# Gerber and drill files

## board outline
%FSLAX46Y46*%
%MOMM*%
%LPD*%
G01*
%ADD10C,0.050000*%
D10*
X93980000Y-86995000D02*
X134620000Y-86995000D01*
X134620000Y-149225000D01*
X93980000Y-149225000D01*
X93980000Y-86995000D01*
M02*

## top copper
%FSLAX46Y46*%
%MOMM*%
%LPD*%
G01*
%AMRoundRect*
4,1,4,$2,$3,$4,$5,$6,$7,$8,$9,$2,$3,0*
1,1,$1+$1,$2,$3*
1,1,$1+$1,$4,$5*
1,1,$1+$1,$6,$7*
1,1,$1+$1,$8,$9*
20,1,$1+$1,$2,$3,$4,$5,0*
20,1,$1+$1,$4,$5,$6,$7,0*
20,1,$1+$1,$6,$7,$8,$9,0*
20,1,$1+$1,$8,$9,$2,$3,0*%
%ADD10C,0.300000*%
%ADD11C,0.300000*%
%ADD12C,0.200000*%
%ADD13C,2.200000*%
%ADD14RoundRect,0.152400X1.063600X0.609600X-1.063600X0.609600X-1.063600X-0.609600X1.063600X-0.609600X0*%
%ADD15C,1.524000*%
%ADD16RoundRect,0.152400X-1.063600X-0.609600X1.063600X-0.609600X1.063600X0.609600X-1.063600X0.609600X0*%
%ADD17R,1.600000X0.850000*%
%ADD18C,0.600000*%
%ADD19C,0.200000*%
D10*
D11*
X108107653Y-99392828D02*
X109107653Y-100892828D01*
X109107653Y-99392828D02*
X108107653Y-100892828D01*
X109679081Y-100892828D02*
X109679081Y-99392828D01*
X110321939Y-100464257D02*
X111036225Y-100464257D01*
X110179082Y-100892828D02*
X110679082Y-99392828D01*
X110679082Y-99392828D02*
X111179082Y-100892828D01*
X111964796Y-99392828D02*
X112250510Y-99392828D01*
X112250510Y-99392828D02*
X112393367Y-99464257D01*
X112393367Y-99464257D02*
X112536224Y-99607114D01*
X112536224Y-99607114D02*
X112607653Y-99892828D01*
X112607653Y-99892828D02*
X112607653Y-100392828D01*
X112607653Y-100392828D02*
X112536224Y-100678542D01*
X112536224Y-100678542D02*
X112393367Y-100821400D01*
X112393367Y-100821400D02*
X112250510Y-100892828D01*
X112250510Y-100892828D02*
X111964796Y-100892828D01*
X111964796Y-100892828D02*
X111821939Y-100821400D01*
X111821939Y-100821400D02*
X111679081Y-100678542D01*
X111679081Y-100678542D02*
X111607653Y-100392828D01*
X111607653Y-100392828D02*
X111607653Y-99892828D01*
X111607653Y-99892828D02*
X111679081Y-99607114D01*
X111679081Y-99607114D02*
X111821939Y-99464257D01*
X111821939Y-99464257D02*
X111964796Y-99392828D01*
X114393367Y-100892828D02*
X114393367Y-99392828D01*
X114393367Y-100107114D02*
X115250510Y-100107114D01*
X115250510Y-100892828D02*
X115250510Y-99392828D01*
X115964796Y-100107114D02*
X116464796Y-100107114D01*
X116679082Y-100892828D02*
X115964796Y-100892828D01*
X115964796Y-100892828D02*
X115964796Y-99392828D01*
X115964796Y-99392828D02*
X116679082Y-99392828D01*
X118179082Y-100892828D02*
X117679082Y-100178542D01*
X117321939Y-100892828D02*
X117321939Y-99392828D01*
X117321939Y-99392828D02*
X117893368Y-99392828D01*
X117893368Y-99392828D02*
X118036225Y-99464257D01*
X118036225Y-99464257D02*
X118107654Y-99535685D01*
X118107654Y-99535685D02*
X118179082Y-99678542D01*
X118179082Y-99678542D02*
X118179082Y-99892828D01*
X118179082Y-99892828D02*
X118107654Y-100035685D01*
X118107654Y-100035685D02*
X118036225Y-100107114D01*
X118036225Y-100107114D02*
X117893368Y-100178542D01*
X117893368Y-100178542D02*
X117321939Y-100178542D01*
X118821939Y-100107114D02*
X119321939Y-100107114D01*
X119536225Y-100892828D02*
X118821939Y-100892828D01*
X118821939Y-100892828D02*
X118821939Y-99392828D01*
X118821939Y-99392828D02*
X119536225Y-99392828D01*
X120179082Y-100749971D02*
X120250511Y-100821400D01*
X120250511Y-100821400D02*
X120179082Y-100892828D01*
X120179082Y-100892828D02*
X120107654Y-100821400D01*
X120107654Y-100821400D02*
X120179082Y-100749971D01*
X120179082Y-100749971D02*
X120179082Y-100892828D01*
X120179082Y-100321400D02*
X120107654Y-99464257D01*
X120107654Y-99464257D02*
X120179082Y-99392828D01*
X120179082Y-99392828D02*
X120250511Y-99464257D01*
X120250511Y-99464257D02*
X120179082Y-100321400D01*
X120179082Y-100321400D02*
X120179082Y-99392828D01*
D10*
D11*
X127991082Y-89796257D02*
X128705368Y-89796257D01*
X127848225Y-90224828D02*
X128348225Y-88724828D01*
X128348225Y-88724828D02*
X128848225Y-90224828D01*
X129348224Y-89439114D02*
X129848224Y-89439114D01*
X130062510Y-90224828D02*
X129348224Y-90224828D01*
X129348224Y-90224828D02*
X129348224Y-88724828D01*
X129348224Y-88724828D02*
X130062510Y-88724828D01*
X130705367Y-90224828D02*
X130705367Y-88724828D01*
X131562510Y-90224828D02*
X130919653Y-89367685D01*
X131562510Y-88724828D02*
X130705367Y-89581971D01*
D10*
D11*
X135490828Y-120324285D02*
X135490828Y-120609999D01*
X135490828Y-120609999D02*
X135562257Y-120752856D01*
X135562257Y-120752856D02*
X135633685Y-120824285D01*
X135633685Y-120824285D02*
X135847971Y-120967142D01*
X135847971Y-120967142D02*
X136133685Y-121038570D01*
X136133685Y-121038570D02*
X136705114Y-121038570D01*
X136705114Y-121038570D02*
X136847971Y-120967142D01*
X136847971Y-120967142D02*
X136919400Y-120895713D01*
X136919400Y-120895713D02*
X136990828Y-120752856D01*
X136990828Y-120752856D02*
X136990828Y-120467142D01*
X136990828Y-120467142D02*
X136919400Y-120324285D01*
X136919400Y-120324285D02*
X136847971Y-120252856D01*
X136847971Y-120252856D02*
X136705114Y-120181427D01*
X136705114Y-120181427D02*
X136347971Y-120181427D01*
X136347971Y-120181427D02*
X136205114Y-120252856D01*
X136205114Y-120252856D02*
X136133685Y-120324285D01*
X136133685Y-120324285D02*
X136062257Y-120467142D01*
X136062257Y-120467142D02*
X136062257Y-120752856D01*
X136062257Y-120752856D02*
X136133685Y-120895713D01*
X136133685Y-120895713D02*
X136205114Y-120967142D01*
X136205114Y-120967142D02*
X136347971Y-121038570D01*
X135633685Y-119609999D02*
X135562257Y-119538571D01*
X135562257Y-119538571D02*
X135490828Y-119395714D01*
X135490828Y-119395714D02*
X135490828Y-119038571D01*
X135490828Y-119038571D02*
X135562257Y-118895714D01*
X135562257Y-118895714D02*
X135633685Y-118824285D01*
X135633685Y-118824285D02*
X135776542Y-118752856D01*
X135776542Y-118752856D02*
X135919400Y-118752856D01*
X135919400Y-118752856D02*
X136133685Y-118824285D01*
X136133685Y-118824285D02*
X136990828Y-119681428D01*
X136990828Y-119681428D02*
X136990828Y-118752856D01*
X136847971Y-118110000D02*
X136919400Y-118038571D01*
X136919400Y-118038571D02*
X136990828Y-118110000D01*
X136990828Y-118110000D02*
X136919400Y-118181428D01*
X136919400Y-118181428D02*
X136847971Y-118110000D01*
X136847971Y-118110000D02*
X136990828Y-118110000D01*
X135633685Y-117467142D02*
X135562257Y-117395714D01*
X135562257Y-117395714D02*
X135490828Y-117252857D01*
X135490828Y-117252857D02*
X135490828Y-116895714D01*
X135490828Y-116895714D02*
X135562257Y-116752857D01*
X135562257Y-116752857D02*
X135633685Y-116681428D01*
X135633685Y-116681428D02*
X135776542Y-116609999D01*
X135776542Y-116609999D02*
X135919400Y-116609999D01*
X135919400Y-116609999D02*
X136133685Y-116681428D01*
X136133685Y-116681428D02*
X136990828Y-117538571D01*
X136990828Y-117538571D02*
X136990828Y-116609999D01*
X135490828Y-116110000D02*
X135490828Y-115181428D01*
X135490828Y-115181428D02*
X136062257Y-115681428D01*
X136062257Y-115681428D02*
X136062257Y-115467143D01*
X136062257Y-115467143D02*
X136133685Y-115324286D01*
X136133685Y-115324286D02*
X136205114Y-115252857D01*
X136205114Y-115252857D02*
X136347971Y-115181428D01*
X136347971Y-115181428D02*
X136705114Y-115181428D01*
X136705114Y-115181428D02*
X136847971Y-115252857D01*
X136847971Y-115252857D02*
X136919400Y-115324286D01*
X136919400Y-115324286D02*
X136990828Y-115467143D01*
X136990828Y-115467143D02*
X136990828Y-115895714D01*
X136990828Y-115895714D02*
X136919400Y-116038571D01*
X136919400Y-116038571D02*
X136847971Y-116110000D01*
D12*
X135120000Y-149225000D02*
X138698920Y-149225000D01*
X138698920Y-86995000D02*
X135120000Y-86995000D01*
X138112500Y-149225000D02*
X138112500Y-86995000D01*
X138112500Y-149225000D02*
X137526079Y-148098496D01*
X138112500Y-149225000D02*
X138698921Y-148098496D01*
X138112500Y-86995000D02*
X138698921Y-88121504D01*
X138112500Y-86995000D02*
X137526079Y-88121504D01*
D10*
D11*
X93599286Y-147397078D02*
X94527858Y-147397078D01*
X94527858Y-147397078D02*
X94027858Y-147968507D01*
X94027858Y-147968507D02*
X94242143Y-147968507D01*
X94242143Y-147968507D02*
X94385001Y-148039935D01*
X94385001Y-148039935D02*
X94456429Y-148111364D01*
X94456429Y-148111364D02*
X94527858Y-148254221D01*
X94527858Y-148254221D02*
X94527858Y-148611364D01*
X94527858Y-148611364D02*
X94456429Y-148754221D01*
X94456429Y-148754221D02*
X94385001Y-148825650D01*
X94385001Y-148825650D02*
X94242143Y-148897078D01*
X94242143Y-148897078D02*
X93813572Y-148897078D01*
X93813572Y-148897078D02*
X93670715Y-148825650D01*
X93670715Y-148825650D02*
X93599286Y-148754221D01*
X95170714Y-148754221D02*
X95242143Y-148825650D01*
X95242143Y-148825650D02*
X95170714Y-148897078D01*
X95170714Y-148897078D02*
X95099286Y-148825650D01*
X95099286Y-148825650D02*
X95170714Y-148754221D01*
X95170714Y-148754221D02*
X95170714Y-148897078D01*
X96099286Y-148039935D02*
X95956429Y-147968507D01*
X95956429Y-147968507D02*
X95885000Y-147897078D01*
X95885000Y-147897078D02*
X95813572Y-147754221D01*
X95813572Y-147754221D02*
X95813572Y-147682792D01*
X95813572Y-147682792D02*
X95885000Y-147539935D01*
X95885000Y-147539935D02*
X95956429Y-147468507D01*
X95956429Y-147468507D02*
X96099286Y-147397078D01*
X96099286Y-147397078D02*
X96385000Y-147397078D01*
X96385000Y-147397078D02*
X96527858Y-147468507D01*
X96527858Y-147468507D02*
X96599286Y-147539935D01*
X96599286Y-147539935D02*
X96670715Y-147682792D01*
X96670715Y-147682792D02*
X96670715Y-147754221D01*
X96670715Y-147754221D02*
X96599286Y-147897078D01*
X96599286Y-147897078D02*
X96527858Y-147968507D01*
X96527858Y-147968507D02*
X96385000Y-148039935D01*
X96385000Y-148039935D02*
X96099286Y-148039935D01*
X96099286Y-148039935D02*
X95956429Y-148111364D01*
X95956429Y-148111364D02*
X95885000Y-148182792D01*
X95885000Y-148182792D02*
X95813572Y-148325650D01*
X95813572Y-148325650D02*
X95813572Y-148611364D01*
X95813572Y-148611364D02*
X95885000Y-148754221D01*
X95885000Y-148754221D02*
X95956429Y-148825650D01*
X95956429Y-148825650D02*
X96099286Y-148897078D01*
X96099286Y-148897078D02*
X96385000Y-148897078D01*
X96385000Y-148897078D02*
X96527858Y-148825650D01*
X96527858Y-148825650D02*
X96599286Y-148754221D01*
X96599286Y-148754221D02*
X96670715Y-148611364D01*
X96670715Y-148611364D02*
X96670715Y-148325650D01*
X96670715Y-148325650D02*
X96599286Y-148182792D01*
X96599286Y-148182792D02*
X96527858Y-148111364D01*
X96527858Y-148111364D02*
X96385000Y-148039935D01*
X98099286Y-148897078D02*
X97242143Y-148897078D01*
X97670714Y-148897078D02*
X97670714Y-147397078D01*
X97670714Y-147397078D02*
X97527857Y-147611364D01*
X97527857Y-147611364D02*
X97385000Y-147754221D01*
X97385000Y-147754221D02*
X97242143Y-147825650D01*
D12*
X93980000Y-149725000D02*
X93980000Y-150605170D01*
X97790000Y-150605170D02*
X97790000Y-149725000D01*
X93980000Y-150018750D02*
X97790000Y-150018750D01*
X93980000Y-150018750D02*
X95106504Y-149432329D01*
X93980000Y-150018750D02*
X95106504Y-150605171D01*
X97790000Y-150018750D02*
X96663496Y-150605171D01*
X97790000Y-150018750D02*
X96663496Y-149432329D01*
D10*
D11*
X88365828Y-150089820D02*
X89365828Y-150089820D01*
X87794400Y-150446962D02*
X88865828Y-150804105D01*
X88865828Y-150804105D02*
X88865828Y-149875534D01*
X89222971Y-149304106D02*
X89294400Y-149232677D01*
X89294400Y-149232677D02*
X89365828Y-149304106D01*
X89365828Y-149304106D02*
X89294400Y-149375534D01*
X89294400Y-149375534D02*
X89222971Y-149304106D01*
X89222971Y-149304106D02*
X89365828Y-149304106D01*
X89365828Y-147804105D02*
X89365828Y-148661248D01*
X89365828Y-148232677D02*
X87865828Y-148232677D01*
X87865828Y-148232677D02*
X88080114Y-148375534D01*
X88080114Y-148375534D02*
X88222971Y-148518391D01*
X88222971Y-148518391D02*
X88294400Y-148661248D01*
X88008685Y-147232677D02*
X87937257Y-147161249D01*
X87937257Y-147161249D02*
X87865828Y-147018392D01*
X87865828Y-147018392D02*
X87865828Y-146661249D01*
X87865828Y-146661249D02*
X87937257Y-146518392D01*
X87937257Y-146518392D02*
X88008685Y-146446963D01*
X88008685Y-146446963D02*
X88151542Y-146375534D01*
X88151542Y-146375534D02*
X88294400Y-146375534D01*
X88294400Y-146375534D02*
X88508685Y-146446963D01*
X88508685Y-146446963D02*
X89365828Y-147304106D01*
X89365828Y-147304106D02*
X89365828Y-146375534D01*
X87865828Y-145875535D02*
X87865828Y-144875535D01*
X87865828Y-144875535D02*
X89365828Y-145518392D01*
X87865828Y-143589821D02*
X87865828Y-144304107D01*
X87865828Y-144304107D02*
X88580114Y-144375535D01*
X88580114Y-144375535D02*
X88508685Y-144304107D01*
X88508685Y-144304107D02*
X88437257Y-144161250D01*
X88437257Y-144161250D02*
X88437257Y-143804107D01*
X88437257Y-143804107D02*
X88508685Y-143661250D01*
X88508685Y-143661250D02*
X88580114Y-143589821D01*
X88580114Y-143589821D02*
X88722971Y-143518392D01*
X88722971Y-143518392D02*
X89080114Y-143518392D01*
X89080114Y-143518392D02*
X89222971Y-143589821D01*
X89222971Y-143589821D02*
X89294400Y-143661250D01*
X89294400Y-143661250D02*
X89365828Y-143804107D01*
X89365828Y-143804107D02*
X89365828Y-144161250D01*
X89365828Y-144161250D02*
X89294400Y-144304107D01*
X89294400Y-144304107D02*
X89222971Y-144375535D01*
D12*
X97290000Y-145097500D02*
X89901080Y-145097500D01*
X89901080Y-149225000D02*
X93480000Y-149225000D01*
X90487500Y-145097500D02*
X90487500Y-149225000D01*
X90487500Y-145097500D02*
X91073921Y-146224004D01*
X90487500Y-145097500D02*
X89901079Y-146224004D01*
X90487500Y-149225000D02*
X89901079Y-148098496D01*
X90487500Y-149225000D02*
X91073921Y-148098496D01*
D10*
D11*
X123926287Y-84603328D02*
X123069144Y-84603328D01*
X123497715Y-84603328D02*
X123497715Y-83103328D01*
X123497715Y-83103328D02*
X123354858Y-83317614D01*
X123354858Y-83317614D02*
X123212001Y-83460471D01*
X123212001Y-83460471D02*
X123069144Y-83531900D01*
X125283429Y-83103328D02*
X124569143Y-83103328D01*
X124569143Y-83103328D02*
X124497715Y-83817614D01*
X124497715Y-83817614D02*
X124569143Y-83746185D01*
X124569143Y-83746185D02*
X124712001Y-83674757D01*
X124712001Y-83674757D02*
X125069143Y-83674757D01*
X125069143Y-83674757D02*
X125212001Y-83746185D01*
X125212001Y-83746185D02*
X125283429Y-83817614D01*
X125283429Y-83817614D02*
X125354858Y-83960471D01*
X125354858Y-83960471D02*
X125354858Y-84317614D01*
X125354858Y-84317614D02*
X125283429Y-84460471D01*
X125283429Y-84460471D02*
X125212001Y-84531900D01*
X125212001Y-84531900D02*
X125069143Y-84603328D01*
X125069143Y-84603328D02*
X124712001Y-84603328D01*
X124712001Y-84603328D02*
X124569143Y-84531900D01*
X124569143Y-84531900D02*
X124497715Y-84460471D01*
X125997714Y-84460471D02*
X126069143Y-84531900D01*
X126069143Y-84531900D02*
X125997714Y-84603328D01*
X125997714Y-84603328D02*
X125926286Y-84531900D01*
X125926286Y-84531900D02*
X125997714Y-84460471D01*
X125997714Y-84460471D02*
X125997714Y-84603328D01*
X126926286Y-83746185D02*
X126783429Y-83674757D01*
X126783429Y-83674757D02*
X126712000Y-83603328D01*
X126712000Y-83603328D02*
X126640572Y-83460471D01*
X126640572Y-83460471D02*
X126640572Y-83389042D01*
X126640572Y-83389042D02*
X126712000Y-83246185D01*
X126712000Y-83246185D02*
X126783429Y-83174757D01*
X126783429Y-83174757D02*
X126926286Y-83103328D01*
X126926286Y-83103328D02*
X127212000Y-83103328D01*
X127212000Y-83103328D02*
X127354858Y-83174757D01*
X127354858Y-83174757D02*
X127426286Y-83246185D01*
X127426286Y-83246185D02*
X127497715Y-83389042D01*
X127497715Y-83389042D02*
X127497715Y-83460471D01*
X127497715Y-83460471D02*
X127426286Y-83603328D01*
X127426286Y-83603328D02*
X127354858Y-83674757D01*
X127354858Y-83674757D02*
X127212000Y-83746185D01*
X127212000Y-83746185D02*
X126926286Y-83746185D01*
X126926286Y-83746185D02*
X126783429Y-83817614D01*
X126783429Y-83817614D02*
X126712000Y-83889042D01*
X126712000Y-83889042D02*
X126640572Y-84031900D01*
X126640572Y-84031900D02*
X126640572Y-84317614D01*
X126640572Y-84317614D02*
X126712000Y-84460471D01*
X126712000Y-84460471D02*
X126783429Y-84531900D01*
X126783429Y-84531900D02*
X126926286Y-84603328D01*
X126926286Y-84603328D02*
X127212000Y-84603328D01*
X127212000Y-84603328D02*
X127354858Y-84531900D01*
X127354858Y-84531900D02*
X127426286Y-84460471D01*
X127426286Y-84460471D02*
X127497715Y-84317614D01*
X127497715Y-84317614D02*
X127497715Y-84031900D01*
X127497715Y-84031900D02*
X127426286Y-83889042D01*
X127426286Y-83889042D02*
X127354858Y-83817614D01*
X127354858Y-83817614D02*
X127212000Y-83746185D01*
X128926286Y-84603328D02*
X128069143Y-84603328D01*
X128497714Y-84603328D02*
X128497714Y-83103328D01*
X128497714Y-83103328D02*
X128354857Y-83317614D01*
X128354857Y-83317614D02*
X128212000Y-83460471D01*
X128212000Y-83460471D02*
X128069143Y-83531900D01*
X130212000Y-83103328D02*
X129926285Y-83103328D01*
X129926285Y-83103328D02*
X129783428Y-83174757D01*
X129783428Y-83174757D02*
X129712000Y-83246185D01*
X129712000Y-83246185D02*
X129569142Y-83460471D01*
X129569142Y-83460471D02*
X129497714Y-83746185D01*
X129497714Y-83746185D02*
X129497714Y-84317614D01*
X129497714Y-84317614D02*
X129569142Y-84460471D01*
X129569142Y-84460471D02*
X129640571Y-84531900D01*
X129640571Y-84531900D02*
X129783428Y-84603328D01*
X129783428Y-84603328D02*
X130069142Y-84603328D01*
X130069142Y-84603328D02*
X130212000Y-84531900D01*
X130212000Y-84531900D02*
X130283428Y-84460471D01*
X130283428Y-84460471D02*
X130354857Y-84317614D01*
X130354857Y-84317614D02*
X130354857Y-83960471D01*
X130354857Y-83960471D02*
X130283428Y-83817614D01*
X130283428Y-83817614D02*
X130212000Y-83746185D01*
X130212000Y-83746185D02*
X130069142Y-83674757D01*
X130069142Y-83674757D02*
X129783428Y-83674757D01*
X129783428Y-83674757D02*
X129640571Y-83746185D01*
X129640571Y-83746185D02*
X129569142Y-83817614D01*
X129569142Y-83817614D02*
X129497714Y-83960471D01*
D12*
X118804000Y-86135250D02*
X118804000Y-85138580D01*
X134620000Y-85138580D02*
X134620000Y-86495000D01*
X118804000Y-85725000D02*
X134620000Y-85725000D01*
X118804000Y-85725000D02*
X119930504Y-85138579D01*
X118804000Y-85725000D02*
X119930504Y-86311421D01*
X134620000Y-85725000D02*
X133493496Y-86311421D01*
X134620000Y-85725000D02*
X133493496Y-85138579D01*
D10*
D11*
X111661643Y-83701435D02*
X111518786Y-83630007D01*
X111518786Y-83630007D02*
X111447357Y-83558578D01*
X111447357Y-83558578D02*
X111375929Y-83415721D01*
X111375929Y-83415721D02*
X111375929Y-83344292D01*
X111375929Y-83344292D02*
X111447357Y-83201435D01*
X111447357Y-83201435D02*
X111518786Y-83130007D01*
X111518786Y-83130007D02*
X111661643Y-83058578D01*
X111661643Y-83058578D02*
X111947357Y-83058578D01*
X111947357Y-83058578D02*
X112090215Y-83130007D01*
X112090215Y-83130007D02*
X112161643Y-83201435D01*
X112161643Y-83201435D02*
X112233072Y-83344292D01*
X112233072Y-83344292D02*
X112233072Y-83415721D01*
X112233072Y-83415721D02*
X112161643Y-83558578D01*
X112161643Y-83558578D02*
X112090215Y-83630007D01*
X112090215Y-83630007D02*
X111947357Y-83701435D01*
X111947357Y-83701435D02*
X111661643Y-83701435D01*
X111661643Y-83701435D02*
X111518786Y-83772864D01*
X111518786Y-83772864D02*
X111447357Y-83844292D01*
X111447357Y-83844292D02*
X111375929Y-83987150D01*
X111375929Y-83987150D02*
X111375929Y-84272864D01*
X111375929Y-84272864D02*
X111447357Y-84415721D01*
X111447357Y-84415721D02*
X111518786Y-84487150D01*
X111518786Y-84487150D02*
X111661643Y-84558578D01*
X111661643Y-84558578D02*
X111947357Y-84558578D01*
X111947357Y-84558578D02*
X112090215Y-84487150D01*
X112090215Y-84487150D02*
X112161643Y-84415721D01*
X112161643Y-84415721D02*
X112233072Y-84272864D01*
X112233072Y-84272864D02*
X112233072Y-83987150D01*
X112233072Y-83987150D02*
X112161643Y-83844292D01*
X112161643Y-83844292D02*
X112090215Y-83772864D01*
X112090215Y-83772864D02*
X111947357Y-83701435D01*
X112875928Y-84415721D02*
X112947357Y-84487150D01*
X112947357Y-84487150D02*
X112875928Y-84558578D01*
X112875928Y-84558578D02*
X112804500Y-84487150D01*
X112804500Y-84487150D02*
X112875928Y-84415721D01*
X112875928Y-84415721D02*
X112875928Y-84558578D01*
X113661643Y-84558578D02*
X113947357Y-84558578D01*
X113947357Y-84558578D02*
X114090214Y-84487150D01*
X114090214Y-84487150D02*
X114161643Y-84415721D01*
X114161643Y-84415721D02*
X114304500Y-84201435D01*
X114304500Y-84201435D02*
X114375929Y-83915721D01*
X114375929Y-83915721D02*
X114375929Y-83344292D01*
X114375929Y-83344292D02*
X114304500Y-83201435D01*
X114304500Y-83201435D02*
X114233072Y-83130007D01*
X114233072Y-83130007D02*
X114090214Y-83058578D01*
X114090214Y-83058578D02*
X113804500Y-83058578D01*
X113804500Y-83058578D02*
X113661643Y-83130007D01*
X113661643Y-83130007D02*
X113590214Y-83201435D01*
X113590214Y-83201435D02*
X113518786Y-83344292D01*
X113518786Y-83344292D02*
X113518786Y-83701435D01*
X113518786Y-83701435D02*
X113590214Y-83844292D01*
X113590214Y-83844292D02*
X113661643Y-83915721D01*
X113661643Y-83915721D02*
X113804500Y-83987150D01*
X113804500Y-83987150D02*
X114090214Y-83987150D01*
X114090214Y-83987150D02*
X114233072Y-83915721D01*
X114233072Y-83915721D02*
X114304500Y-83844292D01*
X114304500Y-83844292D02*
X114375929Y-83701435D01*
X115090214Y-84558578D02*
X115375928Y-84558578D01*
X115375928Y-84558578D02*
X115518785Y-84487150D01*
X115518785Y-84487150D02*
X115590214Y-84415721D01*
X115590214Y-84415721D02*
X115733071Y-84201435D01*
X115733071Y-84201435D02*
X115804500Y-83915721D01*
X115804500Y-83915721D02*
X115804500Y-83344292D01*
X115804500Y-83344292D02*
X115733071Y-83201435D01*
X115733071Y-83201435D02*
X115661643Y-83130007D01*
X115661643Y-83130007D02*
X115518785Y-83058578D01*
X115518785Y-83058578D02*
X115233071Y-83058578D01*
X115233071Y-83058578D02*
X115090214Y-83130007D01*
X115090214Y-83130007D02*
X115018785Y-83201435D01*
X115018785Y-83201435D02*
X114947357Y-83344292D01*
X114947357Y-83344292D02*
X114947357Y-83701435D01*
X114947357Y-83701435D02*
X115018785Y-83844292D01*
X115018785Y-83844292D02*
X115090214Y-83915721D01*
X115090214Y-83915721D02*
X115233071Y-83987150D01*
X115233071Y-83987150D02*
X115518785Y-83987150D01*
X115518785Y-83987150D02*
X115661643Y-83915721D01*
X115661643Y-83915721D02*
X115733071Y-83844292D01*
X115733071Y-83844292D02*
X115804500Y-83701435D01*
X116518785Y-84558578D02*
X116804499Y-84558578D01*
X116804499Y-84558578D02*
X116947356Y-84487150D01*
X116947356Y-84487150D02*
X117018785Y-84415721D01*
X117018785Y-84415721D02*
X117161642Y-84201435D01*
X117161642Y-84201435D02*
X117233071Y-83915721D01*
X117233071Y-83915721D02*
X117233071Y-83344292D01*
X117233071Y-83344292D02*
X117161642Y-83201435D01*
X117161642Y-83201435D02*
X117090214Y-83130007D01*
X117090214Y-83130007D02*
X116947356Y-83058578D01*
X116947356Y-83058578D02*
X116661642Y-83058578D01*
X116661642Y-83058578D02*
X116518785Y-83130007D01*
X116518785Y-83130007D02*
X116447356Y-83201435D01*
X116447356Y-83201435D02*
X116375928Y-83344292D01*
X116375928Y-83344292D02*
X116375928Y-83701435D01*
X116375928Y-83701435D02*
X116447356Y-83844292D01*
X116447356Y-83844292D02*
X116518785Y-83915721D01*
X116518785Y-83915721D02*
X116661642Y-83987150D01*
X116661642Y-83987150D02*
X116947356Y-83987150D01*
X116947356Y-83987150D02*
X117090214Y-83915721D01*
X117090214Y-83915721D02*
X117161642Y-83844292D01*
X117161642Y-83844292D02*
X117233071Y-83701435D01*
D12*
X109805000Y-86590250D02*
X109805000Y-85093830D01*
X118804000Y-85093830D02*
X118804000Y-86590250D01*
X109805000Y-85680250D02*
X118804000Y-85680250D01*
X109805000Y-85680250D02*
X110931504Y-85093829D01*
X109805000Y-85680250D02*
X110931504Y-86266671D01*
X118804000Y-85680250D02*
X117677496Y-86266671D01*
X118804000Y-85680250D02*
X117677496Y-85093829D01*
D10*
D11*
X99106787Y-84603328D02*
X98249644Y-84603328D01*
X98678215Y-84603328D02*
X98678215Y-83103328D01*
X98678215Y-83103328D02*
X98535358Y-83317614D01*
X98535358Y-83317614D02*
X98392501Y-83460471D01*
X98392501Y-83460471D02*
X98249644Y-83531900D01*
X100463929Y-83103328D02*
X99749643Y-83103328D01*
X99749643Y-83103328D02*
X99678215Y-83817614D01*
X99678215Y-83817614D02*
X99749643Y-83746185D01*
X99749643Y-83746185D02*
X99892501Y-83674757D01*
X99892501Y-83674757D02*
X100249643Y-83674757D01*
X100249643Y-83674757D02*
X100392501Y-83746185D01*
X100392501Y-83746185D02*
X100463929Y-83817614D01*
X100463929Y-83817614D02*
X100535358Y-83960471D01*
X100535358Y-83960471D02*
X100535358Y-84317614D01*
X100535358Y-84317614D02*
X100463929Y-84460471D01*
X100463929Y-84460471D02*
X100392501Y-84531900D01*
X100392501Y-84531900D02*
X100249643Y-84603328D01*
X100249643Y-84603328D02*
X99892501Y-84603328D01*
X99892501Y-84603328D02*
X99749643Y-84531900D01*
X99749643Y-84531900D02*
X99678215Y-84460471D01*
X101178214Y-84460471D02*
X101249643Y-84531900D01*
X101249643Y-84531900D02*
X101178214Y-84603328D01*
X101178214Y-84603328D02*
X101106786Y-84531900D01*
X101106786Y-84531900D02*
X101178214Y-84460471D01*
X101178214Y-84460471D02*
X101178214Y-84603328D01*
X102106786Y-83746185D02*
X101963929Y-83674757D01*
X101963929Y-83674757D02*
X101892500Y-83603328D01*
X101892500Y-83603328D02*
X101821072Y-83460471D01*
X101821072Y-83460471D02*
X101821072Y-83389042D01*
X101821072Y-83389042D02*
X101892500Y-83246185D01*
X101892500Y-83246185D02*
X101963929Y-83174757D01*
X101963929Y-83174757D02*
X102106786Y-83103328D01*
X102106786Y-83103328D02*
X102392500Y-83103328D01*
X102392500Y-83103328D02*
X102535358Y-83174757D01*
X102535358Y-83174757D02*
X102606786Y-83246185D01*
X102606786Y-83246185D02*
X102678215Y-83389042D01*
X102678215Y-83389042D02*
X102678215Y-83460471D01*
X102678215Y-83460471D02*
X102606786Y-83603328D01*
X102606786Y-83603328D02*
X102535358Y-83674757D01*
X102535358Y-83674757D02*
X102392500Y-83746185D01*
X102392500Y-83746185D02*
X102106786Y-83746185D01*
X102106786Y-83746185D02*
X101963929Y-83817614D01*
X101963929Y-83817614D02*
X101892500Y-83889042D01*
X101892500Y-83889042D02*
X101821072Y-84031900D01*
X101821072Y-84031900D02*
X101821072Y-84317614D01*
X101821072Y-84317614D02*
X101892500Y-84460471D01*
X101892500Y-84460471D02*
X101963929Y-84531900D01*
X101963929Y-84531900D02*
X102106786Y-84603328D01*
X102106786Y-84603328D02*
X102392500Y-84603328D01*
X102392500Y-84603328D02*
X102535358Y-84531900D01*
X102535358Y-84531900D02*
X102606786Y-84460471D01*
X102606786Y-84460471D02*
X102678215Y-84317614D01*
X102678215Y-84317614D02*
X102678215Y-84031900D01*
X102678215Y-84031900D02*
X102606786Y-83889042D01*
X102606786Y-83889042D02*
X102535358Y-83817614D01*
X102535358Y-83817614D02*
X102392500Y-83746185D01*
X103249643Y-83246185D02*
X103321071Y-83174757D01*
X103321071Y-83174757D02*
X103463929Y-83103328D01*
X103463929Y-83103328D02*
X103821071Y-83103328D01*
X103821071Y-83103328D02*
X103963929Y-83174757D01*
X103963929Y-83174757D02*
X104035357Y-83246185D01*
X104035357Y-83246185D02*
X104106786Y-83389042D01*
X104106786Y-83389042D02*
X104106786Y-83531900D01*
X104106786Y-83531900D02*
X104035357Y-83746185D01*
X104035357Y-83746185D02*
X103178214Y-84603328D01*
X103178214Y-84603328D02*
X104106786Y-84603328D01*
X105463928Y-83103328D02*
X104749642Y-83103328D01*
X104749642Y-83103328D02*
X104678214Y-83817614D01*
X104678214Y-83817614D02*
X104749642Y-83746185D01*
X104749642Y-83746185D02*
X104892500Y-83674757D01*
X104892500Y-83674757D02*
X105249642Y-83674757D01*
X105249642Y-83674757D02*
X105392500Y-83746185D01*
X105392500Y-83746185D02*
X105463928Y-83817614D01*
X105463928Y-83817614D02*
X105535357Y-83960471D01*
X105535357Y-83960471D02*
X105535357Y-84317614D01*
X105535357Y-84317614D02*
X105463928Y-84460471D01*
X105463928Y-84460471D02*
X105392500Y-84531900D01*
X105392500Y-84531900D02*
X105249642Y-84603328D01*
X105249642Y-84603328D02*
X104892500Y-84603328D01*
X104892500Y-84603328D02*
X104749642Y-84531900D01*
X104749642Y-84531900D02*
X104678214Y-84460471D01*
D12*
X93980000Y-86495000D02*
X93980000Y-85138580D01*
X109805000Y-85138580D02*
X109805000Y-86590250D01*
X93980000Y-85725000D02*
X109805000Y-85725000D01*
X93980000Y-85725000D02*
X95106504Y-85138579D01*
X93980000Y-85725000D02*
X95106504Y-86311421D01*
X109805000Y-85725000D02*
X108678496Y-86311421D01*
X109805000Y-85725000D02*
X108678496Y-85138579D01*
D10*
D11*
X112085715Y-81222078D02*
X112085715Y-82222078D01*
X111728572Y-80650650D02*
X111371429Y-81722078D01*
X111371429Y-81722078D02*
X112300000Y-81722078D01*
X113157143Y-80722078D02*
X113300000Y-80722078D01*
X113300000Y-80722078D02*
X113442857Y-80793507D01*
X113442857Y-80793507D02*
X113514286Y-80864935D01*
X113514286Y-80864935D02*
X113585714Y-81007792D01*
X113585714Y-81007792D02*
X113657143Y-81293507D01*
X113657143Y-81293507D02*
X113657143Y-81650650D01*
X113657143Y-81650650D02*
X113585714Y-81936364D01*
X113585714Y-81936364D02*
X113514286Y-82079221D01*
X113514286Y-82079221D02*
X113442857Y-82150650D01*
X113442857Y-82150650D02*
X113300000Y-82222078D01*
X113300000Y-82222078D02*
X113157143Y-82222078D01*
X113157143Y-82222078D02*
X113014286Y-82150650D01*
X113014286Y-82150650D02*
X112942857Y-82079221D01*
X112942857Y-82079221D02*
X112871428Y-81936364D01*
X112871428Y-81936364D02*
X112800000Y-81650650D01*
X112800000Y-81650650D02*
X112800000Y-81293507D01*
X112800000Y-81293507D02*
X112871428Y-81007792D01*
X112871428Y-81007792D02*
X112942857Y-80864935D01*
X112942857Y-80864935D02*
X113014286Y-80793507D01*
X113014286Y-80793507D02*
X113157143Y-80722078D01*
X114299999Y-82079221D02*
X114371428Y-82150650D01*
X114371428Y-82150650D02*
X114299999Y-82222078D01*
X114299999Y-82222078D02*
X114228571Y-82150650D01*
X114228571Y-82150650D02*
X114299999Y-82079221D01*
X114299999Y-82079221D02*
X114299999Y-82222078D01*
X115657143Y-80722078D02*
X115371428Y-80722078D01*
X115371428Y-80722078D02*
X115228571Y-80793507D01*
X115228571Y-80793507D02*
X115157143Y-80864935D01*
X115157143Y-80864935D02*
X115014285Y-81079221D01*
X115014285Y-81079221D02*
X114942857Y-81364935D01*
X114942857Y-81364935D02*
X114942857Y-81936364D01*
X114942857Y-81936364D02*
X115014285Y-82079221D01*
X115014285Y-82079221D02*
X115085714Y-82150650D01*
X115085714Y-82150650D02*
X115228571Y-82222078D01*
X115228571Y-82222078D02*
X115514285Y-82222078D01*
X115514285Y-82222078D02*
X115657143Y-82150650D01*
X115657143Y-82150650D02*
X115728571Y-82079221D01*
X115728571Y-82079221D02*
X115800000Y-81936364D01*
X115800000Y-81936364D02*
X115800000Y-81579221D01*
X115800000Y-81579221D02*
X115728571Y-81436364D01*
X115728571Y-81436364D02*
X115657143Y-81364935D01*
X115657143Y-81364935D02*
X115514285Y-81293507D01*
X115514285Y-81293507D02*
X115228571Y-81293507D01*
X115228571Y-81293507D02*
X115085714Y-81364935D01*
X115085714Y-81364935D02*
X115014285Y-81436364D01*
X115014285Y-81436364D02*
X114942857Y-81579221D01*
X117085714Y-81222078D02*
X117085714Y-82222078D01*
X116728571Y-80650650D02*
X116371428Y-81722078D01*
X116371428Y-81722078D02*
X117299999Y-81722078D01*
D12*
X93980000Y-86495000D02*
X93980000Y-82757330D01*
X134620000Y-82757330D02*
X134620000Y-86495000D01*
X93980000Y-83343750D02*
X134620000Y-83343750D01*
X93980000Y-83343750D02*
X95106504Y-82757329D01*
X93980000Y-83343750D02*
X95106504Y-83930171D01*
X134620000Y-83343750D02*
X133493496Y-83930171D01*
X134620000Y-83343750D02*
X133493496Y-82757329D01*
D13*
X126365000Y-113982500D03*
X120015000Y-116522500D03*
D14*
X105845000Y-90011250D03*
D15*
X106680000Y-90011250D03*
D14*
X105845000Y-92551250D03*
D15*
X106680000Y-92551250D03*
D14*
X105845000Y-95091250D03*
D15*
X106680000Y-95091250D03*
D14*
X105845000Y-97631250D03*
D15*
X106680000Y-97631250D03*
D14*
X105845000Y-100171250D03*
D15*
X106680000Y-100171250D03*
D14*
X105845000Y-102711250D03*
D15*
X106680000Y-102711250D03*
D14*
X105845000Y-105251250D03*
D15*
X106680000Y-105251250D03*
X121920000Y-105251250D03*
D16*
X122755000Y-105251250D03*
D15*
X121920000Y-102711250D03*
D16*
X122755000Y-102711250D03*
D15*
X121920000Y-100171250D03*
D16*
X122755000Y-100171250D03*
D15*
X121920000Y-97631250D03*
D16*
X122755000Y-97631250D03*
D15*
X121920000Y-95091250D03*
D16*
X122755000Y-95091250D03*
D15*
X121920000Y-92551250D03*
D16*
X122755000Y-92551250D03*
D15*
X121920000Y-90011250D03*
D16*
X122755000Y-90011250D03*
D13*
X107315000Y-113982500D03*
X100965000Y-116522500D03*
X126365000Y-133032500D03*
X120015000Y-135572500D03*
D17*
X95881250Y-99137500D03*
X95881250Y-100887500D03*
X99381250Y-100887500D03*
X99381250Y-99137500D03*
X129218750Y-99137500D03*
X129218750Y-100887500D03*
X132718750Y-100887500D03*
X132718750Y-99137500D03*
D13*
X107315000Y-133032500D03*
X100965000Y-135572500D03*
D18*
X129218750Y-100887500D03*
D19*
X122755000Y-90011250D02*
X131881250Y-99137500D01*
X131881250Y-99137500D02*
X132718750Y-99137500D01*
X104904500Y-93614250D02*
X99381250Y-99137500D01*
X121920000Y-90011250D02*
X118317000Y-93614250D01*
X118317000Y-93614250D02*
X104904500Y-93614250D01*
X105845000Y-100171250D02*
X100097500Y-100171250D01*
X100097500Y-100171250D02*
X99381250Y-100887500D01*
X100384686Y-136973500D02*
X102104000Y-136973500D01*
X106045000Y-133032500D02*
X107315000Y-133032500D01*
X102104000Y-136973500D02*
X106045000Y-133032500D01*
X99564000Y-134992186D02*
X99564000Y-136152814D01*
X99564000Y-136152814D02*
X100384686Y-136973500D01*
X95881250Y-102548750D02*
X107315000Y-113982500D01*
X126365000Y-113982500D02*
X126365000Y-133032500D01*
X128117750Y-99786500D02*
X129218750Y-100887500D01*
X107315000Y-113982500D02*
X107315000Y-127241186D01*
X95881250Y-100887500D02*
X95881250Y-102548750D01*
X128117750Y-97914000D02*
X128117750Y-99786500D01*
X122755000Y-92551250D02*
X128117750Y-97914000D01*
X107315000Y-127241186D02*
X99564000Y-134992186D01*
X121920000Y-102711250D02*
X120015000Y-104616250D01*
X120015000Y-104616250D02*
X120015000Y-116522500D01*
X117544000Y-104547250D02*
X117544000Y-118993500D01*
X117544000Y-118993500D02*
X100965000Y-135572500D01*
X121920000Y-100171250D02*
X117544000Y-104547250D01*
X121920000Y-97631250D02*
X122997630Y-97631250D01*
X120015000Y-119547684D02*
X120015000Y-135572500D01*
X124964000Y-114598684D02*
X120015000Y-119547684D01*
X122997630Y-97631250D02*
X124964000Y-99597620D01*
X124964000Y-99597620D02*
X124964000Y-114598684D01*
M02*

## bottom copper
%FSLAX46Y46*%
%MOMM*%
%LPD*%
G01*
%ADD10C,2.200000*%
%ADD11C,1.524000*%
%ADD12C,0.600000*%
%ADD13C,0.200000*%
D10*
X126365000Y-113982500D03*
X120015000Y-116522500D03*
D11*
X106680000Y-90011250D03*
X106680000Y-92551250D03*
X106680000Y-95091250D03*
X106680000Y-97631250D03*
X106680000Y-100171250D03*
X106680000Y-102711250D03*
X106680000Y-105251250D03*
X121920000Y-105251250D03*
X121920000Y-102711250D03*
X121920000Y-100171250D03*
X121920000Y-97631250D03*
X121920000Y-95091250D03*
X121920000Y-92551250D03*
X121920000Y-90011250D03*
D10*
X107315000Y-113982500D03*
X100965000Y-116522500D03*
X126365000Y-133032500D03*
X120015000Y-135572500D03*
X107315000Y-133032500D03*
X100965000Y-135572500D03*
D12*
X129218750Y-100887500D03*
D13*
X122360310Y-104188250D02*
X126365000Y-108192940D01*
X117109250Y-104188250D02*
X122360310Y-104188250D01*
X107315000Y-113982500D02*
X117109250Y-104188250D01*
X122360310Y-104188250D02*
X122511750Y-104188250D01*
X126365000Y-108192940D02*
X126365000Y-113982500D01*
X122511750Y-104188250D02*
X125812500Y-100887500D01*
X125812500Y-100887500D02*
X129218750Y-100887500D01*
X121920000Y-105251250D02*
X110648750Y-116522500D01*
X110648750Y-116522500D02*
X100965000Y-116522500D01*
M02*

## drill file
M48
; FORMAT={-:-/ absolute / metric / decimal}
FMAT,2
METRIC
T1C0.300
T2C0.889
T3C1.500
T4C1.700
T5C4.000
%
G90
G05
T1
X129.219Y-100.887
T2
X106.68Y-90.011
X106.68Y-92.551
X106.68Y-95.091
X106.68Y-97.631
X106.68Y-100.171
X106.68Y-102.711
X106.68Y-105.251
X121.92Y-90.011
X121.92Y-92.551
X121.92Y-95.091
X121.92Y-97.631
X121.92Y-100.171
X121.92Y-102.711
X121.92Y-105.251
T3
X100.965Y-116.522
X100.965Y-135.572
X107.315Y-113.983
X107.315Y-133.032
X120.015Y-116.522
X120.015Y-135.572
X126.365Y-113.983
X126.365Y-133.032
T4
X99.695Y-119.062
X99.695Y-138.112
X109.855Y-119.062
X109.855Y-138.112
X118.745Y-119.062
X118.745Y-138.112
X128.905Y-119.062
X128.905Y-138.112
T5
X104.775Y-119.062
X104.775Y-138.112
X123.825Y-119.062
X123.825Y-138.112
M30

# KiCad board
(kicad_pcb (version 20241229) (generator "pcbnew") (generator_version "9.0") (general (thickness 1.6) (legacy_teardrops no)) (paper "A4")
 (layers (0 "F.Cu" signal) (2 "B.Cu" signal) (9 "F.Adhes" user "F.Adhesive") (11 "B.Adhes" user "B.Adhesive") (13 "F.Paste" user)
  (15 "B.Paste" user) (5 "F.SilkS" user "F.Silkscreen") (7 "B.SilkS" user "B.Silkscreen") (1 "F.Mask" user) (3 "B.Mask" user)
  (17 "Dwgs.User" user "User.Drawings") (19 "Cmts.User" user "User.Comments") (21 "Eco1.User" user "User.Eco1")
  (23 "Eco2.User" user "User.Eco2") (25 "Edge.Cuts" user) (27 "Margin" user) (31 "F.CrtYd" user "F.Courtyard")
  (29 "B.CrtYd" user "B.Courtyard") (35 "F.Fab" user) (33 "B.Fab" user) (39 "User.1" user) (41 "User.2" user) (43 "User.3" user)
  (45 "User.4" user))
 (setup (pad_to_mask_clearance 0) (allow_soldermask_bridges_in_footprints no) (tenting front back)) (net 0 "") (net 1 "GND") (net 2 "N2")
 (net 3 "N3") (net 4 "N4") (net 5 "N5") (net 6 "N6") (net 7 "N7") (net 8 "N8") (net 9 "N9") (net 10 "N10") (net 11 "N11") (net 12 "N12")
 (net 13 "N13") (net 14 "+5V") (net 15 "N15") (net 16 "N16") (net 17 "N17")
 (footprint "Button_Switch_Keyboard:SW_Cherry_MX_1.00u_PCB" (layer "F.Cu") (at 126.365 113.9825)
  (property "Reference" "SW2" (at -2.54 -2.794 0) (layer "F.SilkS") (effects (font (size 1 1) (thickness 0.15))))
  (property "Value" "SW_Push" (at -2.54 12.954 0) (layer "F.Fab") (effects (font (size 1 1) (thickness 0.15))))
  (pad "" np_thru_hole circle (at -7.62 5.08) (size 1.7 1.7) (drill 1.7) (layers "*.Cu" "*.Mask"))
  (pad "" np_thru_hole circle (at -2.54 5.08) (size 4 4) (drill 4) (layers "*.Cu" "*.Mask"))
  (pad "" np_thru_hole circle (at 2.54 5.08) (size 1.7 1.7) (drill 1.7) (layers "*.Cu" "*.Mask"))
  (pad "1" thru_hole circle (at 0 0) (size 2.2 2.2) (drill 1.5) (layers "*.Cu" "*.Mask") (remove_unused_layers no) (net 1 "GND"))
  (pad "2" thru_hole circle (at -6.35 2.54) (size 2.2 2.2) (drill 1.5) (layers "*.Cu" "*.Mask") (remove_unused_layers no) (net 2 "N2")))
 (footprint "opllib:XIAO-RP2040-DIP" (layer "F.Cu") (at 114.3 97.63125)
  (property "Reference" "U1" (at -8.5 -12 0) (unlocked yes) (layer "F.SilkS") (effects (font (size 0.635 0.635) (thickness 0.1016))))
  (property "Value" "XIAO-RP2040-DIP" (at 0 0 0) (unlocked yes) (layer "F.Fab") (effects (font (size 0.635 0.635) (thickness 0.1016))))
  (pad "1" smd roundrect (at -8.455 -7.62 180) (size 2.432 1.524) (layers "F.Cu" "F.Mask") (roundrect_rratio 0.1) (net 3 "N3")
   (thermal_bridge_angle 45))
  (pad "1" thru_hole circle (at -7.62 -7.62 180) (size 1.524 1.524) (drill 0.889) (layers "*.Cu" "*.Mask") (remove_unused_layers no)
   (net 3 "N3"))
  (pad "2" smd roundrect (at -8.455 -5.08 180) (size 2.432 1.524) (layers "F.Cu" "F.Mask") (roundrect_rratio 0.1) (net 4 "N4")
   (thermal_bridge_angle 45))
  (pad "2" thru_hole circle (at -7.62 -5.08 180) (size 1.524 1.524) (drill 0.889) (layers "*.Cu" "*.Mask") (remove_unused_layers no)
   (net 4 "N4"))
  (pad "3" smd roundrect (at -8.455 -2.54 180) (size 2.432 1.524) (layers "F.Cu" "F.Mask") (roundrect_rratio 0.1) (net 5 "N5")
   (thermal_bridge_angle 45))
  (pad "3" thru_hole circle (at -7.62 -2.54 180) (size 1.524 1.524) (drill 0.889) (layers "*.Cu" "*.Mask") (remove_unused_layers no)
   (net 5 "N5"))
  (pad "4" smd roundrect (at -8.455 0 180) (size 2.432 1.524) (layers "F.Cu" "F.Mask") (roundrect_rratio 0.1) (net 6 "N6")
   (thermal_bridge_angle 45))
  (pad "4" thru_hole circle (at -7.62 0 180) (size 1.524 1.524) (drill 0.889) (layers "*.Cu" "*.Mask") (remove_unused_layers no)
   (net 6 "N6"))
  (pad "5" smd roundrect (at -8.455 2.54 180) (size 2.432 1.524) (layers "F.Cu" "F.Mask") (roundrect_rratio 0.1) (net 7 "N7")
   (thermal_bridge_angle 45))
  (pad "5" thru_hole circle (at -7.62 2.54 180) (size 1.524 1.524) (drill 0.889) (layers "*.Cu" "*.Mask") (remove_unused_layers no)
   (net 7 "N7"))
  (pad "6" smd roundrect (at -8.455 5.08 180) (size 2.432 1.524) (layers "F.Cu" "F.Mask") (roundrect_rratio 0.1) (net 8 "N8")
   (thermal_bridge_angle 45))
  (pad "6" thru_hole circle (at -7.62 5.08 180) (size 1.524 1.524) (drill 0.889) (layers "*.Cu" "*.Mask") (remove_unused_layers no)
   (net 8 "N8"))
  (pad "7" smd roundrect (at -8.455 7.62 180) (size 2.432 1.524) (layers "F.Cu" "F.Mask") (roundrect_rratio 0.1) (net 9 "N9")
   (thermal_bridge_angle 45))
  (pad "7" thru_hole circle (at -7.62 7.62 180) (size 1.524 1.524) (drill 0.889) (layers "*.Cu" "*.Mask") (remove_unused_layers no)
   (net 9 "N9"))
  (pad "8" thru_hole circle (at 7.62 7.62) (size 1.524 1.524) (drill 0.889) (layers "*.Cu" "*.Mask") (remove_unused_layers no)
   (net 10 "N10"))
  (pad "8" smd roundrect (at 8.455 7.62) (size 2.432 1.524) (layers "F.Cu" "F.Mask") (roundrect_rratio 0.1) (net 10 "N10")
   (thermal_bridge_angle 45))
  (pad "9" thru_hole circle (at 7.62 5.08) (size 1.524 1.524) (drill 0.889) (layers "*.Cu" "*.Mask") (remove_unused_layers no) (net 2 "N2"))
  (pad "9" smd roundrect (at 8.455 5.08) (size 2.432 1.524) (layers "F.Cu" "F.Mask") (roundrect_rratio 0.1) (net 2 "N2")
   (thermal_bridge_angle 45))
  (pad "10" thru_hole circle (at 7.62 2.54) (size 1.524 1.524) (drill 0.889) (layers "*.Cu" "*.Mask") (remove_unused_layers no)
   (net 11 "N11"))
  (pad "10" smd roundrect (at 8.455 2.54) (size 2.432 1.524) (layers "F.Cu" "F.Mask") (roundrect_rratio 0.1) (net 11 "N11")
   (thermal_bridge_angle 45))
  (pad "11" thru_hole circle (at 7.62 0) (size 1.524 1.524) (drill 0.889) (layers "*.Cu" "*.Mask") (remove_unused_layers no) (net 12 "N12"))
  (pad "11" smd roundrect (at 8.455 0) (size 2.432 1.524) (layers "F.Cu" "F.Mask") (roundrect_rratio 0.1) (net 12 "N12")
   (thermal_bridge_angle 45))
  (pad "12" thru_hole circle (at 7.62 -2.54) (size 1.524 1.524) (drill 0.889) (layers "*.Cu" "*.Mask") (remove_unused_layers no)
   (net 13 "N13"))
  (pad "12" smd roundrect (at 8.455 -2.54) (size 2.432 1.524) (layers "F.Cu" "F.Mask") (roundrect_rratio 0.1) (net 13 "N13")
   (thermal_bridge_angle 45))
  (pad "13" thru_hole circle (at 7.62 -5.08) (size 1.524 1.524) (drill 0.889) (layers "*.Cu" "*.Mask") (remove_unused_layers no)
   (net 1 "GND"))
  (pad "13" smd roundrect (at 8.455 -5.08) (size 2.432 1.524) (layers "F.Cu" "F.Mask") (roundrect_rratio 0.1) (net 1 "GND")
   (thermal_bridge_angle 45))
  (pad "14" thru_hole circle (at 7.62 -7.62) (size 1.524 1.524) (drill 0.889) (layers "*.Cu" "*.Mask") (remove_unused_layers no)
   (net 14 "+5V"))
  (pad "14" smd roundrect (at 8.455 -7.62) (size 2.432 1.524) (layers "F.Cu" "F.Mask") (roundrect_rratio 0.1) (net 14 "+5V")
   (thermal_bridge_angle 45)))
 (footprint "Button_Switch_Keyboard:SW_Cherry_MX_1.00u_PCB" (layer "F.Cu") (at 107.315 113.9825)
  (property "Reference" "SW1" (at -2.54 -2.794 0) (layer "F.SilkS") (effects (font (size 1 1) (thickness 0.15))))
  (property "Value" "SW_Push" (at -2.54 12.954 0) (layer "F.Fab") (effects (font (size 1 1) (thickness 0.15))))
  (pad "" np_thru_hole circle (at -7.62 5.08) (size 1.7 1.7) (drill 1.7) (layers "*.Cu" "*.Mask"))
  (pad "" np_thru_hole circle (at -2.54 5.08) (size 4 4) (drill 4) (layers "*.Cu" "*.Mask"))
  (pad "" np_thru_hole circle (at 2.54 5.08) (size 1.7 1.7) (drill 1.7) (layers "*.Cu" "*.Mask"))
  (pad "1" thru_hole circle (at 0 0) (size 2.2 2.2) (drill 1.5) (layers "*.Cu" "*.Mask") (remove_unused_layers no) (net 1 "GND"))
  (pad "2" thru_hole circle (at -6.35 2.54) (size 2.2 2.2) (drill 1.5) (layers "*.Cu" "*.Mask") (remove_unused_layers no) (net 10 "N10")))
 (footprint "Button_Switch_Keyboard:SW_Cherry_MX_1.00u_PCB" (layer "F.Cu") (at 126.365 133.0325)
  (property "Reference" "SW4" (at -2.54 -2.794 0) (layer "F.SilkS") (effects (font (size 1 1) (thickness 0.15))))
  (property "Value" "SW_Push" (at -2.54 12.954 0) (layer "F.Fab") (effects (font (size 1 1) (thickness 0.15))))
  (pad "" np_thru_hole circle (at -7.62 5.08) (size 1.7 1.7) (drill 1.7) (layers "*.Cu" "*.Mask"))
  (pad "" np_thru_hole circle (at -2.54 5.08) (size 4 4) (drill 4) (layers "*.Cu" "*.Mask"))
  (pad "" np_thru_hole circle (at 2.54 5.08) (size 1.7 1.7) (drill 1.7) (layers "*.Cu" "*.Mask"))
  (pad "1" thru_hole circle (at 0 0) (size 2.2 2.2) (drill 1.5) (layers "*.Cu" "*.Mask") (remove_unused_layers no) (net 1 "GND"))
  (pad "2" thru_hole circle (at -6.35 2.54) (size 2.2 2.2) (drill 1.5) (layers "*.Cu" "*.Mask") (remove_unused_layers no) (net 12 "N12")))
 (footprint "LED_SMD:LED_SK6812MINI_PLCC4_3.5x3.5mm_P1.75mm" (layer "F.Cu") (at 97.63125 100.0125)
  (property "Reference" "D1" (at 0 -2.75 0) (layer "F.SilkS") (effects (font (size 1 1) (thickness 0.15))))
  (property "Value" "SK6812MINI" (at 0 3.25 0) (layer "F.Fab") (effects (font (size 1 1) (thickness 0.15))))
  (pad "1" smd rect (at -1.75 -0.875) (size 1.6 0.85) (layers "F.Cu" "F.Mask" "F.Paste") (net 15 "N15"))
  (pad "2" smd rect (at -1.75 0.875) (size 1.6 0.85) (layers "F.Cu" "F.Mask" "F.Paste") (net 1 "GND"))
  (pad "3" smd rect (at 1.75 0.875) (size 1.6 0.85) (layers "F.Cu" "F.Mask" "F.Paste") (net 7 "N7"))
  (pad "4" smd rect (at 1.75 -0.875) (size 1.6 0.85) (layers "F.Cu" "F.Mask" "F.Paste") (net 14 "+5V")))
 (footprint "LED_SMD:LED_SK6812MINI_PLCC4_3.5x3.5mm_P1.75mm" (layer "F.Cu") (at 130.96875 100.0125)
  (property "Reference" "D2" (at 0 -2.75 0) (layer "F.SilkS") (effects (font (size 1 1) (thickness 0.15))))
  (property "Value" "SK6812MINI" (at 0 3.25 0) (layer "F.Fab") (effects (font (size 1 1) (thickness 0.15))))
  (pad "1" smd rect (at -1.75 -0.875) (size 1.6 0.85) (layers "F.Cu" "F.Mask" "F.Paste") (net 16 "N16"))
  (pad "2" smd rect (at -1.75 0.875) (size 1.6 0.85) (layers "F.Cu" "F.Mask" "F.Paste") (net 1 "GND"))
  (pad "3" smd rect (at 1.75 0.875) (size 1.6 0.85) (layers "F.Cu" "F.Mask" "F.Paste") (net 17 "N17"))
  (pad "4" smd rect (at 1.75 -0.875) (size 1.6 0.85) (layers "F.Cu" "F.Mask" "F.Paste") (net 14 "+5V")))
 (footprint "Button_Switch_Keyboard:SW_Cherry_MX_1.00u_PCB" (layer "F.Cu") (at 107.315 133.0325)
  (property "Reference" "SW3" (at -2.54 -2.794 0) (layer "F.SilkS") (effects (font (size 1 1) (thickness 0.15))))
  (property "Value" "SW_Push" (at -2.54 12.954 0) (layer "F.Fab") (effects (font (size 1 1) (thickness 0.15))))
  (pad "" np_thru_hole circle (at -7.62 5.08) (size 1.7 1.7) (drill 1.7) (layers "*.Cu" "*.Mask"))
  (pad "" np_thru_hole circle (at -2.54 5.08) (size 4 4) (drill 4) (layers "*.Cu" "*.Mask"))
  (pad "" np_thru_hole circle (at 2.54 5.08) (size 1.7 1.7) (drill 1.7) (layers "*.Cu" "*.Mask"))
  (pad "1" thru_hole circle (at 0 0) (size 2.2 2.2) (drill 1.5) (layers "*.Cu" "*.Mask") (remove_unused_layers no) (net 1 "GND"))
  (pad "2" thru_hole circle (at -6.35 2.54) (size 2.2 2.2) (drill 1.5) (layers "*.Cu" "*.Mask") (remove_unused_layers no) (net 11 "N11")))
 (gr_rect (start 93.98 86.995) (end 134.62 149.225) (stroke (width 0.05) (type default)) (fill no) (layer "Edge.Cuts"))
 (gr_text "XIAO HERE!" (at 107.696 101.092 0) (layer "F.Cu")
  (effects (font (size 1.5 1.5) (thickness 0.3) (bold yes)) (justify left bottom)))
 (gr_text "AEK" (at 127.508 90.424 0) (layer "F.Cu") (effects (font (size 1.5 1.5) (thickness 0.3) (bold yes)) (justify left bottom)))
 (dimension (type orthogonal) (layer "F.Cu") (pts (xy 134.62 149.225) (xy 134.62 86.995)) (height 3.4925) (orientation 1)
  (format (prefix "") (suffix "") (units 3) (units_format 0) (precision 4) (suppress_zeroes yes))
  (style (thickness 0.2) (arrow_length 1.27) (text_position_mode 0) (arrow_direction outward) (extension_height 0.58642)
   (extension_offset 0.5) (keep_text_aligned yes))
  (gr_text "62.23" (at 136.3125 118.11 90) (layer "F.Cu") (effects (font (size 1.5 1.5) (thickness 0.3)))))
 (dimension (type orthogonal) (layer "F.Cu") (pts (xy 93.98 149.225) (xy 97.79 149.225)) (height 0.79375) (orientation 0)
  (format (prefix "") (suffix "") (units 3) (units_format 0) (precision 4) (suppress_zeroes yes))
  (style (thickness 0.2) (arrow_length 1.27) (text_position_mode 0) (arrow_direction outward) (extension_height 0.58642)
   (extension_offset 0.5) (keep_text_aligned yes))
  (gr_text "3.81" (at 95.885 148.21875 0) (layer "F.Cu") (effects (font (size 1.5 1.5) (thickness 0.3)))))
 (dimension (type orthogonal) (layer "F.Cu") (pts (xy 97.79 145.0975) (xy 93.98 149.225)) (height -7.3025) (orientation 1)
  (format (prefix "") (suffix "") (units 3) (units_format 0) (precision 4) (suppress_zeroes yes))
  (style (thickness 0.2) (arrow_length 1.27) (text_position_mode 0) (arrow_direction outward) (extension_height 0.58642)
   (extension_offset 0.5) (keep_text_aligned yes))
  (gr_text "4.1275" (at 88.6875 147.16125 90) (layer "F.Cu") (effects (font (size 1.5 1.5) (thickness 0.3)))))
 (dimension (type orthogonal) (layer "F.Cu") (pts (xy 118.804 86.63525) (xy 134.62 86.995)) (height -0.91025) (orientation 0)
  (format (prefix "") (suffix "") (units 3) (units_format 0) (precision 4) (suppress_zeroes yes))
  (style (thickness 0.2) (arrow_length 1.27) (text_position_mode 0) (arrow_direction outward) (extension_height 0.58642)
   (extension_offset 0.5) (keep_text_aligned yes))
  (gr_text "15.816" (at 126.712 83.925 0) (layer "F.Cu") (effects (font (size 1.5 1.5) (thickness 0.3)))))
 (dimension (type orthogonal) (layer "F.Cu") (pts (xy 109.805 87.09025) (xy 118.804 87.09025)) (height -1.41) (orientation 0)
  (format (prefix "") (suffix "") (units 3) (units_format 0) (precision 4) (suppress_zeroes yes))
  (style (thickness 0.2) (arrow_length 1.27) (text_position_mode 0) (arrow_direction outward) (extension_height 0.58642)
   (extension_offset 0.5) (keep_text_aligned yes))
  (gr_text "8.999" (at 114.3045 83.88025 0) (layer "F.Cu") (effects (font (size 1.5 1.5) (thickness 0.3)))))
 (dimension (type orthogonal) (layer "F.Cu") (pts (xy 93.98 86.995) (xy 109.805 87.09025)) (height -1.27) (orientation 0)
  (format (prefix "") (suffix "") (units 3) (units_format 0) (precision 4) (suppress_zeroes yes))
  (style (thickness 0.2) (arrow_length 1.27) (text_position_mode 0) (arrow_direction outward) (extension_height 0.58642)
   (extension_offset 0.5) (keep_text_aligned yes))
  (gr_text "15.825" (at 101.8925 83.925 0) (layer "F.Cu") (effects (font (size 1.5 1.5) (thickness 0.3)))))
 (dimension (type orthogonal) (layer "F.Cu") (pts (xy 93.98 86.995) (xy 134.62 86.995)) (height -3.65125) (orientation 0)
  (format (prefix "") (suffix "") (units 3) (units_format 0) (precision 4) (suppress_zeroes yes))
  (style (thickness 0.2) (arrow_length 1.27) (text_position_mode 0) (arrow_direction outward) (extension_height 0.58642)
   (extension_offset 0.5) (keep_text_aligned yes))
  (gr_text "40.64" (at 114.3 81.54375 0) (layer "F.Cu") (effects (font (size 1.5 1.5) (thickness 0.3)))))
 (segment (start 122.755 90.01125) (end 131.88125 99.1375) (width 0.2) (layer "F.Cu") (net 14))
 (segment (start 131.88125 99.1375) (end 132.71875 99.1375) (width 0.2) (layer "F.Cu") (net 14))
 (segment (start 104.9045 93.61425) (end 99.38125 99.1375) (width 0.2) (layer "F.Cu") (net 14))
 (segment (start 121.92 90.01125) (end 118.317 93.61425) (width 0.2) (layer "F.Cu") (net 14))
 (segment (start 118.317 93.61425) (end 104.9045 93.61425) (width 0.2) (layer "F.Cu") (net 14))
 (segment (start 105.845 100.17125) (end 100.0975 100.17125) (width 0.2) (layer "F.Cu") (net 7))
 (segment (start 100.0975 100.17125) (end 99.38125 100.8875) (width 0.2) (layer "F.Cu") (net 7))
 (segment (start 100.384686 136.9735) (end 102.104 136.9735) (width 0.2) (layer "F.Cu") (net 1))
 (segment (start 106.045 133.0325) (end 107.315 133.0325) (width 0.2) (layer "F.Cu") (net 1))
 (segment (start 102.104 136.9735) (end 106.045 133.0325) (width 0.2) (layer "F.Cu") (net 1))
 (segment (start 99.564 134.992186) (end 99.564 136.152814) (width 0.2) (layer "F.Cu") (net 1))
 (segment (start 99.564 136.152814) (end 100.384686 136.9735) (width 0.2) (layer "F.Cu") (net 1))
 (segment (start 95.88125 102.54875) (end 107.315 113.9825) (width 0.2) (layer "F.Cu") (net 1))
 (segment (start 126.365 113.9825) (end 126.365 133.0325) (width 0.2) (layer "F.Cu") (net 1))
 (segment (start 128.11775 99.7865) (end 129.21875 100.8875) (width 0.2) (layer "F.Cu") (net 1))
 (segment (start 107.315 113.9825) (end 107.315 127.241186) (width 0.2) (layer "F.Cu") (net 1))
 (segment (start 95.88125 100.8875) (end 95.88125 102.54875) (width 0.2) (layer "F.Cu") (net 1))
 (segment (start 128.11775 97.914) (end 128.11775 99.7865) (width 0.2) (layer "F.Cu") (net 1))
 (segment (start 122.755 92.55125) (end 128.11775 97.914) (width 0.2) (layer "F.Cu") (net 1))
 (segment (start 107.315 127.241186) (end 99.564 134.992186) (width 0.2) (layer "F.Cu") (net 1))
 (via (at 129.21875 100.8875) (size 0.6) (drill 0.3) (layers "F.Cu" "B.Cu") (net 1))
 (segment (start 122.36031 104.18825) (end 126.365 108.19294) (width 0.2) (layer "B.Cu") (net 1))
 (segment (start 117.10925 104.18825) (end 122.36031 104.18825) (width 0.2) (layer "B.Cu") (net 1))
 (segment (start 107.315 113.9825) (end 117.10925 104.18825) (width 0.2) (layer "B.Cu") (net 1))
 (segment (start 122.36031 104.18825) (end 122.51175 104.18825) (width 0.2) (layer "B.Cu") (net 1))
 (segment (start 126.365 108.19294) (end 126.365 113.9825) (width 0.2) (layer "B.Cu") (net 1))
 (segment (start 122.51175 104.18825) (end 125.8125 100.8875) (width 0.2) (layer "B.Cu") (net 1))
 (segment (start 125.8125 100.8875) (end 129.21875 100.8875) (width 0.2) (layer "B.Cu") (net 1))
 (segment (start 121.92 105.25125) (end 110.64875 116.5225) (width 0.2) (layer "B.Cu") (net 10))
 (segment (start 110.64875 116.5225) (end 100.965 116.5225) (width 0.2) (layer "B.Cu") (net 10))
 (segment (start 121.92 102.71125) (end 120.015 104.61625) (width 0.2) (layer "F.Cu") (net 2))
 (segment (start 120.015 104.61625) (end 120.015 116.5225) (width 0.2) (layer "F.Cu") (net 2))
 (segment (start 117.544 104.54725) (end 117.544 118.9935) (width 0.2) (layer "F.Cu") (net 11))
 (segment (start 117.544 118.9935) (end 100.965 135.5725) (width 0.2) (layer "F.Cu") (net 11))
 (segment (start 121.92 100.17125) (end 117.544 104.54725) (width 0.2) (layer "F.Cu") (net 11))
 (segment (start 121.92 97.63125) (end 122.99763 97.63125) (width 0.2) (layer "F.Cu") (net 12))
 (segment (start 120.015 119.547684) (end 120.015 135.5725) (width 0.2) (layer "F.Cu") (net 12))
 (segment (start 124.964 114.598684) (end 120.015 119.547684) (width 0.2) (layer "F.Cu") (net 12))
 (segment (start 122.99763 97.63125) (end 124.964 99.59762) (width 0.2) (layer "F.Cu") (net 12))
 (segment (start 124.964 99.59762) (end 124.964 114.598684) (width 0.2) (layer "F.Cu") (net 12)))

